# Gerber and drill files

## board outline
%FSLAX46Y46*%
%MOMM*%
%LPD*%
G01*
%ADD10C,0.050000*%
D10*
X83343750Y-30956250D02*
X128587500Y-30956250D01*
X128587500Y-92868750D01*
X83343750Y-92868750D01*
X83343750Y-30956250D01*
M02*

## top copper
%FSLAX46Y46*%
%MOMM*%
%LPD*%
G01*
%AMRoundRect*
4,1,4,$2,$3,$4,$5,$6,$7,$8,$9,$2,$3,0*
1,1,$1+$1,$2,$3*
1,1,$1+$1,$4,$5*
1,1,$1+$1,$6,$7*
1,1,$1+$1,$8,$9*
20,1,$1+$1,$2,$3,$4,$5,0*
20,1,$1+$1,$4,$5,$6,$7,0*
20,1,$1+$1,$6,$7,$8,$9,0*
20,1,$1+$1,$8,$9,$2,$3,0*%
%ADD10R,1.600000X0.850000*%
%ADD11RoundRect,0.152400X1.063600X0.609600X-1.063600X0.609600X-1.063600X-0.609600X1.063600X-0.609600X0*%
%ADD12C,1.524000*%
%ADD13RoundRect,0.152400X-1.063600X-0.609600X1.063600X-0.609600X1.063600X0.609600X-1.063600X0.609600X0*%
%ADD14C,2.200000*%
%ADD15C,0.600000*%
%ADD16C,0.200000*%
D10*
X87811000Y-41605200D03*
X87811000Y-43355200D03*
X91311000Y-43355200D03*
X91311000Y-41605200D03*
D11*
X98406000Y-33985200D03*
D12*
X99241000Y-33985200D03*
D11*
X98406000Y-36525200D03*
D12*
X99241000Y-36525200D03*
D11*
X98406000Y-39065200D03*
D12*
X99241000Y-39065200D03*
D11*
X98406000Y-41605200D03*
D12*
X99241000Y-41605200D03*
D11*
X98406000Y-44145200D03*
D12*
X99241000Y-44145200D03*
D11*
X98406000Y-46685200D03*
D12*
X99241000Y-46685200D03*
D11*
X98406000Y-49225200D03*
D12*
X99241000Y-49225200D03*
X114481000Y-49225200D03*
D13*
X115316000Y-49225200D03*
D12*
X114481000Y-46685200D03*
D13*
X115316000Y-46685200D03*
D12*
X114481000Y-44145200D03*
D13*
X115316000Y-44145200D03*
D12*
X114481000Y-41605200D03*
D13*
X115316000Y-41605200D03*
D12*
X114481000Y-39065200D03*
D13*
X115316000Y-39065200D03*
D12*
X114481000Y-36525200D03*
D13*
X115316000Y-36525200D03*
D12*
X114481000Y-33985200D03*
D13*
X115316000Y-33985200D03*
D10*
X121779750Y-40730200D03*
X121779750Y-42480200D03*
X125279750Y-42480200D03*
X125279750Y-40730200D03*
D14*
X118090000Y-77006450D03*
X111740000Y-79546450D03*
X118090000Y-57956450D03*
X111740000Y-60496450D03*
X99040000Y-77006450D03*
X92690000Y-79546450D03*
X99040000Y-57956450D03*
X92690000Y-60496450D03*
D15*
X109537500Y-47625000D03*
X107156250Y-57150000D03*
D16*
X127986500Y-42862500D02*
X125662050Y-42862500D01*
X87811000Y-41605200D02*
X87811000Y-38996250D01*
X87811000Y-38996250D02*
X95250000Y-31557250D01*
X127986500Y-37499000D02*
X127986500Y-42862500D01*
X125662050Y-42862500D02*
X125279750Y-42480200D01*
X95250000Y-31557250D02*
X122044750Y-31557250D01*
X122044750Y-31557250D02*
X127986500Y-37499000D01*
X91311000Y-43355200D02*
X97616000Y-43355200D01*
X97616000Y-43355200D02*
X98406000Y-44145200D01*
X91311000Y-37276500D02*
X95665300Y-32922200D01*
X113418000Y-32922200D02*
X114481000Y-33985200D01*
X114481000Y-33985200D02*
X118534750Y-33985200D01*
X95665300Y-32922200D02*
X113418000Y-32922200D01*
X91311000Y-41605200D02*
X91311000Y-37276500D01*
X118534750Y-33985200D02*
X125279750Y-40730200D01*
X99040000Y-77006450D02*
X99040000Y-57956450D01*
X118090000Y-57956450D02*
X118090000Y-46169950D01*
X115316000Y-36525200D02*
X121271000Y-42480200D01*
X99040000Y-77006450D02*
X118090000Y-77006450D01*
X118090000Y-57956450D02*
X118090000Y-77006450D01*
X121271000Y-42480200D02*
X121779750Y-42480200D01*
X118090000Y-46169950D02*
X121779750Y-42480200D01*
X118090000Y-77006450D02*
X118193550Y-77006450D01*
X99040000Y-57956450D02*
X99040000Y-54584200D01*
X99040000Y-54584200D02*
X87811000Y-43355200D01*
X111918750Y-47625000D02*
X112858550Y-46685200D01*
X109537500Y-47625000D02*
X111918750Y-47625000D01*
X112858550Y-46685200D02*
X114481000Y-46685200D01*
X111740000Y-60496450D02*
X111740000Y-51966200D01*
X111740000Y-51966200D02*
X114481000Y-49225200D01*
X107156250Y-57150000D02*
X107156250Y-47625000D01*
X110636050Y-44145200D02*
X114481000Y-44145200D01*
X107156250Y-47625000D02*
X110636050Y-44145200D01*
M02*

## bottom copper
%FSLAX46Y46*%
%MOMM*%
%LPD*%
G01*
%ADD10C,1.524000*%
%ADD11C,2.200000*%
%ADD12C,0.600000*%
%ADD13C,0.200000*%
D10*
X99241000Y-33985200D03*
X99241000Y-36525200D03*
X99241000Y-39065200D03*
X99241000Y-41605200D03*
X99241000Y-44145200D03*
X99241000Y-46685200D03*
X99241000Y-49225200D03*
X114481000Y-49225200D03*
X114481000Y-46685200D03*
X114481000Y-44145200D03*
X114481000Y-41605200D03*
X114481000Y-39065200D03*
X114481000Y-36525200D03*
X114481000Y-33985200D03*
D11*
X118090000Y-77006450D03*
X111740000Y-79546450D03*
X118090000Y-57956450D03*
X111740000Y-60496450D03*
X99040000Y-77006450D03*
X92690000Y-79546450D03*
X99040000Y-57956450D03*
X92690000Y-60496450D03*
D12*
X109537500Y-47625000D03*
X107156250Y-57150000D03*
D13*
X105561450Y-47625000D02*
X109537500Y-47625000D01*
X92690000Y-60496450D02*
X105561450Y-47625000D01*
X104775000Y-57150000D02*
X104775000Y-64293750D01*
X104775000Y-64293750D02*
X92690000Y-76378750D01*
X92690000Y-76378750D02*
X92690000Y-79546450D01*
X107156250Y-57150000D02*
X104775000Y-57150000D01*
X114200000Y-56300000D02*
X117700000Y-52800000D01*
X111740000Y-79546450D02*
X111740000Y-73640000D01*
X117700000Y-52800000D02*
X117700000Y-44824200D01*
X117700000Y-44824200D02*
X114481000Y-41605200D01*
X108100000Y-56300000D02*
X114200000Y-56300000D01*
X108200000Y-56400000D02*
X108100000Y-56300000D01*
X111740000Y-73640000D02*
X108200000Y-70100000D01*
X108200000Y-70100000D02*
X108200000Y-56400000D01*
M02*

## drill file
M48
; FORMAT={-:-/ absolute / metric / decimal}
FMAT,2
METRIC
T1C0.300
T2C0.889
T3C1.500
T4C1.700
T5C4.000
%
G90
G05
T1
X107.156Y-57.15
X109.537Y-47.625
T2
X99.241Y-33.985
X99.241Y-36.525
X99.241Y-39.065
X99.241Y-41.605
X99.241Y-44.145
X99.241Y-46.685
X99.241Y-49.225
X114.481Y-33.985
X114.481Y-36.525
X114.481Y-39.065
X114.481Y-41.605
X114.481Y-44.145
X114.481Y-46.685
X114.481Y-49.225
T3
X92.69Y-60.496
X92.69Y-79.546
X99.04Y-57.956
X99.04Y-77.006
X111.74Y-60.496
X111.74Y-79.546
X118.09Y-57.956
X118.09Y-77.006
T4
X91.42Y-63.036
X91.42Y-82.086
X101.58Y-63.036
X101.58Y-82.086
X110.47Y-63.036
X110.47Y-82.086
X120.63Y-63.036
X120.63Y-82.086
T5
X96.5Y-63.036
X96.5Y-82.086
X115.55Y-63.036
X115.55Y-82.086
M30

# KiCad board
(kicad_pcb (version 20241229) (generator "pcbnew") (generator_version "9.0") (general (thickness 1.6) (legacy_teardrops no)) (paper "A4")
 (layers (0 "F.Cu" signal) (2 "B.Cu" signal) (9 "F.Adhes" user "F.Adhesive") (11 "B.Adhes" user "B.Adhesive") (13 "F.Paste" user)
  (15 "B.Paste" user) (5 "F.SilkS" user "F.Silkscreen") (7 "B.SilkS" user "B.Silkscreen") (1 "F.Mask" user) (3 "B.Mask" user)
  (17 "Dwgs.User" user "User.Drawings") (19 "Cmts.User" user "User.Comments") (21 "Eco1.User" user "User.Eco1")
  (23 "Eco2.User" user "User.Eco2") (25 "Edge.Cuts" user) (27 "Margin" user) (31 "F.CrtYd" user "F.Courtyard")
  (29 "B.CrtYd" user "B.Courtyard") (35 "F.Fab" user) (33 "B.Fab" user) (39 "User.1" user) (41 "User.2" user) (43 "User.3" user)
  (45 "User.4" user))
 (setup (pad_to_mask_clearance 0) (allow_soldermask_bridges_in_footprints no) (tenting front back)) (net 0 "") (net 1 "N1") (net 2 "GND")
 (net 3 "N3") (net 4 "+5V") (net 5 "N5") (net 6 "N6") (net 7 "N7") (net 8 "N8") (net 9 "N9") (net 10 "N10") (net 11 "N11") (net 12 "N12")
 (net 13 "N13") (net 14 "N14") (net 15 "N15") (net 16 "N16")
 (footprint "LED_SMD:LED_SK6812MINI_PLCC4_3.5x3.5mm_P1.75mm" (layer "F.Cu") (at 89.561 42.4802)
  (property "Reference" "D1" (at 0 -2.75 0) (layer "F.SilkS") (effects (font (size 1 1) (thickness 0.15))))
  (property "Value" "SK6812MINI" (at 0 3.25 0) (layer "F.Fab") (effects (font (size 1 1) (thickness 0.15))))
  (pad "1" smd rect (at -1.75 -0.875) (size 1.6 0.85) (layers "F.Cu" "F.Mask" "F.Paste") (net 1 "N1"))
  (pad "2" smd rect (at -1.75 0.875) (size 1.6 0.85) (layers "F.Cu" "F.Mask" "F.Paste") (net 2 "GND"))
  (pad "3" smd rect (at 1.75 0.875) (size 1.6 0.85) (layers "F.Cu" "F.Mask" "F.Paste") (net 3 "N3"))
  (pad "4" smd rect (at 1.75 -0.875) (size 1.6 0.85) (layers "F.Cu" "F.Mask" "F.Paste") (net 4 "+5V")))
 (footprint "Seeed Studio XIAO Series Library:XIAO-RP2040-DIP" (layer "F.Cu") (at 106.861 41.6052)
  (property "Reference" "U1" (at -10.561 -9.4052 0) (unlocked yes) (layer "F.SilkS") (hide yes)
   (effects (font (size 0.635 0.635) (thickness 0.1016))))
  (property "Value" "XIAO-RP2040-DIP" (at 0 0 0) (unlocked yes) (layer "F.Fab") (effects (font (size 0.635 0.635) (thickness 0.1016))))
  (pad "1" smd roundrect (at -8.455 -7.62 180) (size 2.432 1.524) (layers "F.Cu" "F.Mask") (roundrect_rratio 0.1) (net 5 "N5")
   (thermal_bridge_angle 45))
  (pad "1" thru_hole circle (at -7.62 -7.62 180) (size 1.524 1.524) (drill 0.889) (layers "*.Cu" "*.Mask") (remove_unused_layers no)
   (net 5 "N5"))
  (pad "2" smd roundrect (at -8.455 -5.08 180) (size 2.432 1.524) (layers "F.Cu" "F.Mask") (roundrect_rratio 0.1) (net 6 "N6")
   (thermal_bridge_angle 45))
  (pad "2" thru_hole circle (at -7.62 -5.08 180) (size 1.524 1.524) (drill 0.889) (layers "*.Cu" "*.Mask") (remove_unused_layers no)
   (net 6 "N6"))
  (pad "3" smd roundrect (at -8.455 -2.54 180) (size 2.432 1.524) (layers "F.Cu" "F.Mask") (roundrect_rratio 0.1) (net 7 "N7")
   (thermal_bridge_angle 45))
  (pad "3" thru_hole circle (at -7.62 -2.54 180) (size 1.524 1.524) (drill 0.889) (layers "*.Cu" "*.Mask") (remove_unused_layers no)
   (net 7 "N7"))
  (pad "4" smd roundrect (at -8.455 0 180) (size 2.432 1.524) (layers "F.Cu" "F.Mask") (roundrect_rratio 0.1) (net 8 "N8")
   (thermal_bridge_angle 45))
  (pad "4" thru_hole circle (at -7.62 0 180) (size 1.524 1.524) (drill 0.889) (layers "*.Cu" "*.Mask") (remove_unused_layers no)
   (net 8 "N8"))
  (pad "5" smd roundrect (at -8.455 2.54 180) (size 2.432 1.524) (layers "F.Cu" "F.Mask") (roundrect_rratio 0.1) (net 3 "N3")
   (thermal_bridge_angle 45))
  (pad "5" thru_hole circle (at -7.62 2.54 180) (size 1.524 1.524) (drill 0.889) (layers "*.Cu" "*.Mask") (remove_unused_layers no)
   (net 3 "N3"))
  (pad "6" smd roundrect (at -8.455 5.08 180) (size 2.432 1.524) (layers "F.Cu" "F.Mask") (roundrect_rratio 0.1) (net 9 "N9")
   (thermal_bridge_angle 45))
  (pad "6" thru_hole circle (at -7.62 5.08 180) (size 1.524 1.524) (drill 0.889) (layers "*.Cu" "*.Mask") (remove_unused_layers no)
   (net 9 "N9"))
  (pad "7" smd roundrect (at -8.455 7.62 180) (size 2.432 1.524) (layers "F.Cu" "F.Mask") (roundrect_rratio 0.1) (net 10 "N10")
   (thermal_bridge_angle 45))
  (pad "7" thru_hole circle (at -7.62 7.62 180) (size 1.524 1.524) (drill 0.889) (layers "*.Cu" "*.Mask") (remove_unused_layers no)
   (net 10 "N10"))
  (pad "8" thru_hole circle (at 7.62 7.62) (size 1.524 1.524) (drill 0.889) (layers "*.Cu" "*.Mask") (remove_unused_layers no)
   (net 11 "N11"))
  (pad "8" smd roundrect (at 8.455 7.62) (size 2.432 1.524) (layers "F.Cu" "F.Mask") (roundrect_rratio 0.1) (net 11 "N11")
   (thermal_bridge_angle 45))
  (pad "9" thru_hole circle (at 7.62 5.08) (size 1.524 1.524) (drill 0.889) (layers "*.Cu" "*.Mask") (remove_unused_layers no)
   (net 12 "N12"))
  (pad "9" smd roundrect (at 8.455 5.08) (size 2.432 1.524) (layers "F.Cu" "F.Mask") (roundrect_rratio 0.1) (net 12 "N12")
   (thermal_bridge_angle 45))
  (pad "10" thru_hole circle (at 7.62 2.54) (size 1.524 1.524) (drill 0.889) (layers "*.Cu" "*.Mask") (remove_unused_layers no)
   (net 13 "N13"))
  (pad "10" smd roundrect (at 8.455 2.54) (size 2.432 1.524) (layers "F.Cu" "F.Mask") (roundrect_rratio 0.1) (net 13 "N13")
   (thermal_bridge_angle 45))
  (pad "11" thru_hole circle (at 7.62 0) (size 1.524 1.524) (drill 0.889) (layers "*.Cu" "*.Mask") (remove_unused_layers no) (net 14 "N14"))
  (pad "11" smd roundrect (at 8.455 0) (size 2.432 1.524) (layers "F.Cu" "F.Mask") (roundrect_rratio 0.1) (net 14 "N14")
   (thermal_bridge_angle 45))
  (pad "12" thru_hole circle (at 7.62 -2.54) (size 1.524 1.524) (drill 0.889) (layers "*.Cu" "*.Mask") (remove_unused_layers no)
   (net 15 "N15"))
  (pad "12" smd roundrect (at 8.455 -2.54) (size 2.432 1.524) (layers "F.Cu" "F.Mask") (roundrect_rratio 0.1) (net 15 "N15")
   (thermal_bridge_angle 45))
  (pad "13" thru_hole circle (at 7.62 -5.08) (size 1.524 1.524) (drill 0.889) (layers "*.Cu" "*.Mask") (remove_unused_layers no)
   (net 2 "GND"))
  (pad "13" smd roundrect (at 8.455 -5.08) (size 2.432 1.524) (layers "F.Cu" "F.Mask") (roundrect_rratio 0.1) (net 2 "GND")
   (thermal_bridge_angle 45))
  (pad "14" thru_hole circle (at 7.62 -7.62) (size 1.524 1.524) (drill 0.889) (layers "*.Cu" "*.Mask") (remove_unused_layers no)
   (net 4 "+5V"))
  (pad "14" smd roundrect (at 8.455 -7.62) (size 2.432 1.524) (layers "F.Cu" "F.Mask") (roundrect_rratio 0.1) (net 4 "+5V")
   (thermal_bridge_angle 45)))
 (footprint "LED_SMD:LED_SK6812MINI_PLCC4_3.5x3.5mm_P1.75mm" (layer "F.Cu") (at 123.52975 41.6052)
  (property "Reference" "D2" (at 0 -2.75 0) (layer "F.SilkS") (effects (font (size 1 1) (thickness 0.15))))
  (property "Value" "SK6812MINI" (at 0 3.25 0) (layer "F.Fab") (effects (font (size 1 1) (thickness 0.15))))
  (pad "1" smd rect (at -1.75 -0.875) (size 1.6 0.85) (layers "F.Cu" "F.Mask" "F.Paste") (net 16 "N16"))
  (pad "2" smd rect (at -1.75 0.875) (size 1.6 0.85) (layers "F.Cu" "F.Mask" "F.Paste") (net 2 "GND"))
  (pad "3" smd rect (at 1.75 0.875) (size 1.6 0.85) (layers "F.Cu" "F.Mask" "F.Paste") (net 1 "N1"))
  (pad "4" smd rect (at 1.75 -0.875) (size 1.6 0.85) (layers "F.Cu" "F.Mask" "F.Paste") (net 4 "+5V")))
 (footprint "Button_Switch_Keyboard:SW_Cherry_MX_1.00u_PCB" (layer "F.Cu") (at 118.09 77.00645)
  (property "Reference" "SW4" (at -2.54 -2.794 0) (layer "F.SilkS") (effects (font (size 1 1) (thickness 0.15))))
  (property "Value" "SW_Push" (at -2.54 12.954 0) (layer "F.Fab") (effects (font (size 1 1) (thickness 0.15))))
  (pad "" np_thru_hole circle (at -7.62 5.08) (size 1.7 1.7) (drill 1.7) (layers "*.Cu" "*.Mask"))
  (pad "" np_thru_hole circle (at -2.54 5.08) (size 4 4) (drill 4) (layers "*.Cu" "*.Mask"))
  (pad "" np_thru_hole circle (at 2.54 5.08) (size 1.7 1.7) (drill 1.7) (layers "*.Cu" "*.Mask"))
  (pad "1" thru_hole circle (at 0 0) (size 2.2 2.2) (drill 1.5) (layers "*.Cu" "*.Mask") (remove_unused_layers no) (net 2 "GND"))
  (pad "2" thru_hole circle (at -6.35 2.54) (size 2.2 2.2) (drill 1.5) (layers "*.Cu" "*.Mask") (remove_unused_layers no) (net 14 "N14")))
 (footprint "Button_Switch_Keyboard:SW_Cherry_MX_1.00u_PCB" (layer "F.Cu") (at 118.09 57.95645)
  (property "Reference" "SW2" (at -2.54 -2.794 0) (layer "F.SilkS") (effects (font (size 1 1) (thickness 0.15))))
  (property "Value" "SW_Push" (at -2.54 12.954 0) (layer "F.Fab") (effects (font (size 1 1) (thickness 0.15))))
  (pad "" np_thru_hole circle (at -7.62 5.08) (size 1.7 1.7) (drill 1.7) (layers "*.Cu" "*.Mask"))
  (pad "" np_thru_hole circle (at -2.54 5.08) (size 4 4) (drill 4) (layers "*.Cu" "*.Mask"))
  (pad "" np_thru_hole circle (at 2.54 5.08) (size 1.7 1.7) (drill 1.7) (layers "*.Cu" "*.Mask"))
  (pad "1" thru_hole circle (at 0 0) (size 2.2 2.2) (drill 1.5) (layers "*.Cu" "*.Mask") (remove_unused_layers no) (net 2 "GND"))
  (pad "2" thru_hole circle (at -6.35 2.54) (size 2.2 2.2) (drill 1.5) (layers "*.Cu" "*.Mask") (remove_unused_layers no) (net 11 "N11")))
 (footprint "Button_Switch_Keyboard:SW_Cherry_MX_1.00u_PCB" (layer "F.Cu") (at 99.04 77.00645)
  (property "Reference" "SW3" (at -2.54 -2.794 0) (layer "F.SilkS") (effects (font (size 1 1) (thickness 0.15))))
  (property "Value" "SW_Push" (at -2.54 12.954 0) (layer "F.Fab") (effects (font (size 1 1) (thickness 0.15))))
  (pad "" np_thru_hole circle (at -7.62 5.08) (size 1.7 1.7) (drill 1.7) (layers "*.Cu" "*.Mask"))
  (pad "" np_thru_hole circle (at -2.54 5.08) (size 4 4) (drill 4) (layers "*.Cu" "*.Mask"))
  (pad "" np_thru_hole circle (at 2.54 5.08) (size 1.7 1.7) (drill 1.7) (layers "*.Cu" "*.Mask"))
  (pad "1" thru_hole circle (at 0 0) (size 2.2 2.2) (drill 1.5) (layers "*.Cu" "*.Mask") (remove_unused_layers no) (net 2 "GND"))
  (pad "2" thru_hole circle (at -6.35 2.54) (size 2.2 2.2) (drill 1.5) (layers "*.Cu" "*.Mask") (remove_unused_layers no) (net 13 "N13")))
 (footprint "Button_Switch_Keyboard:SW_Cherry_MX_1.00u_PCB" (layer "F.Cu") (at 99.04 57.95645)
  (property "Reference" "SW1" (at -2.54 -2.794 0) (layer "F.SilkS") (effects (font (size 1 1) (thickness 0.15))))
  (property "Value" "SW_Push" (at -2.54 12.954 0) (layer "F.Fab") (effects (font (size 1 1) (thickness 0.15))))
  (pad "" np_thru_hole circle (at -7.62 5.08) (size 1.7 1.7) (drill 1.7) (layers "*.Cu" "*.Mask"))
  (pad "" np_thru_hole circle (at -2.54 5.08) (size 4 4) (drill 4) (layers "*.Cu" "*.Mask"))
  (pad "" np_thru_hole circle (at 2.54 5.08) (size 1.7 1.7) (drill 1.7) (layers "*.Cu" "*.Mask"))
  (pad "1" thru_hole circle (at 0 0) (size 2.2 2.2) (drill 1.5) (layers "*.Cu" "*.Mask") (remove_unused_layers no) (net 2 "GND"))
  (pad "2" thru_hole circle (at -6.35 2.54) (size 2.2 2.2) (drill 1.5) (layers "*.Cu" "*.Mask") (remove_unused_layers no) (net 12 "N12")))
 (gr_rect (start 83.34375 30.95625) (end 128.5875 92.86875) (stroke (width 0.05) (type default)) (fill no) (layer "Edge.Cuts"))
 (segment (start 127.9865 42.8625) (end 125.66205 42.8625) (width 0.2) (layer "F.Cu") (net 1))
 (segment (start 87.811 41.6052) (end 87.811 38.99625) (width 0.2) (layer "F.Cu") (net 1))
 (segment (start 87.811 38.99625) (end 95.25 31.55725) (width 0.2) (layer "F.Cu") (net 1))
 (segment (start 127.9865 37.499) (end 127.9865 42.8625) (width 0.2) (layer "F.Cu") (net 1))
 (segment (start 125.66205 42.8625) (end 125.27975 42.4802) (width 0.2) (layer "F.Cu") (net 1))
 (segment (start 95.25 31.55725) (end 122.04475 31.55725) (width 0.2) (layer "F.Cu") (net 1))
 (segment (start 122.04475 31.55725) (end 127.9865 37.499) (width 0.2) (layer "F.Cu") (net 1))
 (segment (start 91.311 43.3552) (end 97.616 43.3552) (width 0.2) (layer "F.Cu") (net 3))
 (segment (start 97.616 43.3552) (end 98.406 44.1452) (width 0.2) (layer "F.Cu") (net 3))
 (segment (start 91.311 37.2765) (end 95.6653 32.9222) (width 0.2) (layer "F.Cu") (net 4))
 (segment (start 113.418 32.9222) (end 114.481 33.9852) (width 0.2) (layer "F.Cu") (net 4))
 (segment (start 114.481 33.9852) (end 118.53475 33.9852) (width 0.2) (layer "F.Cu") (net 4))
 (segment (start 95.6653 32.9222) (end 113.418 32.9222) (width 0.2) (layer "F.Cu") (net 4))
 (segment (start 91.311 41.6052) (end 91.311 37.2765) (width 0.2) (layer "F.Cu") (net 4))
 (segment (start 118.53475 33.9852) (end 125.27975 40.7302) (width 0.2) (layer "F.Cu") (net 4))
 (segment (start 99.04 77.00645) (end 99.04 57.95645) (width 0.2) (layer "F.Cu") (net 2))
 (segment (start 118.09 57.95645) (end 118.09 46.16995) (width 0.2) (layer "F.Cu") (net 2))
 (segment (start 115.316 36.5252) (end 121.271 42.4802) (width 0.2) (layer "F.Cu") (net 2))
 (segment (start 99.04 77.00645) (end 118.09 77.00645) (width 0.2) (layer "F.Cu") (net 2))
 (segment (start 118.09 57.95645) (end 118.09 77.00645) (width 0.2) (layer "F.Cu") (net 2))
 (segment (start 121.271 42.4802) (end 121.77975 42.4802) (width 0.2) (layer "F.Cu") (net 2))
 (segment (start 118.09 46.16995) (end 121.77975 42.4802) (width 0.2) (layer "F.Cu") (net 2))
 (segment (start 118.09 77.00645) (end 118.19355 77.00645) (width 0.2) (layer "F.Cu") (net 2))
 (segment (start 99.04 57.95645) (end 99.04 54.5842) (width 0.2) (layer "F.Cu") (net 2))
 (segment (start 99.04 54.5842) (end 87.811 43.3552) (width 0.2) (layer "F.Cu") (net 2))
 (segment (start 111.91875 47.625) (end 112.85855 46.6852) (width 0.2) (layer "F.Cu") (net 12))
 (segment (start 109.5375 47.625) (end 111.91875 47.625) (width 0.2) (layer "F.Cu") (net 12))
 (segment (start 112.85855 46.6852) (end 114.481 46.6852) (width 0.2) (layer "F.Cu") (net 12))
 (via (at 109.5375 47.625) (size 0.6) (drill 0.3) (layers "F.Cu" "B.Cu") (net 12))
 (segment (start 105.56145 47.625) (end 109.5375 47.625) (width 0.2) (layer "B.Cu") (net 12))
 (segment (start 92.69 60.49645) (end 105.56145 47.625) (width 0.2) (layer "B.Cu") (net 12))
 (segment (start 111.74 60.49645) (end 111.74 51.9662) (width 0.2) (layer "F.Cu") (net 11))
 (segment (start 111.74 51.9662) (end 114.481 49.2252) (width 0.2) (layer "F.Cu") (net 11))
 (segment (start 107.15625 57.15) (end 107.15625 47.625) (width 0.2) (layer "F.Cu") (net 13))
 (segment (start 110.63605 44.1452) (end 114.481 44.1452) (width 0.2) (layer "F.Cu") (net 13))
 (segment (start 107.15625 47.625) (end 110.63605 44.1452) (width 0.2) (layer "F.Cu") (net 13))
 (via (at 107.15625 57.15) (size 0.6) (drill 0.3) (layers "F.Cu" "B.Cu") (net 13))
 (segment (start 104.775 57.15) (end 104.775 64.29375) (width 0.2) (layer "B.Cu") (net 13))
 (segment (start 104.775 64.29375) (end 92.69 76.37875) (width 0.2) (layer "B.Cu") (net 13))
 (segment (start 92.69 76.37875) (end 92.69 79.54645) (width 0.2) (layer "B.Cu") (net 13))
 (segment (start 107.15625 57.15) (end 104.775 57.15) (width 0.2) (layer "B.Cu") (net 13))
 (segment (start 114.2 56.3) (end 117.7 52.8) (width 0.2) (layer "B.Cu") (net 14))
 (segment (start 111.74 79.54645) (end 111.74 73.64) (width 0.2) (layer "B.Cu") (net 14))
 (segment (start 117.7 52.8) (end 117.7 44.8242) (width 0.2) (layer "B.Cu") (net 14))
 (segment (start 117.7 44.8242) (end 114.481 41.6052) (width 0.2) (layer "B.Cu") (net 14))
 (segment (start 108.1 56.3) (end 114.2 56.3) (width 0.2) (layer "B.Cu") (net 14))
 (segment (start 108.2 56.4) (end 108.1 56.3) (width 0.2) (layer "B.Cu") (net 14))
 (segment (start 111.74 73.64) (end 108.2 70.1) (width 0.2) (layer "B.Cu") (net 14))
 (segment (start 108.2 70.1) (end 108.2 56.4) (width 0.2) (layer "B.Cu") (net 14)))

